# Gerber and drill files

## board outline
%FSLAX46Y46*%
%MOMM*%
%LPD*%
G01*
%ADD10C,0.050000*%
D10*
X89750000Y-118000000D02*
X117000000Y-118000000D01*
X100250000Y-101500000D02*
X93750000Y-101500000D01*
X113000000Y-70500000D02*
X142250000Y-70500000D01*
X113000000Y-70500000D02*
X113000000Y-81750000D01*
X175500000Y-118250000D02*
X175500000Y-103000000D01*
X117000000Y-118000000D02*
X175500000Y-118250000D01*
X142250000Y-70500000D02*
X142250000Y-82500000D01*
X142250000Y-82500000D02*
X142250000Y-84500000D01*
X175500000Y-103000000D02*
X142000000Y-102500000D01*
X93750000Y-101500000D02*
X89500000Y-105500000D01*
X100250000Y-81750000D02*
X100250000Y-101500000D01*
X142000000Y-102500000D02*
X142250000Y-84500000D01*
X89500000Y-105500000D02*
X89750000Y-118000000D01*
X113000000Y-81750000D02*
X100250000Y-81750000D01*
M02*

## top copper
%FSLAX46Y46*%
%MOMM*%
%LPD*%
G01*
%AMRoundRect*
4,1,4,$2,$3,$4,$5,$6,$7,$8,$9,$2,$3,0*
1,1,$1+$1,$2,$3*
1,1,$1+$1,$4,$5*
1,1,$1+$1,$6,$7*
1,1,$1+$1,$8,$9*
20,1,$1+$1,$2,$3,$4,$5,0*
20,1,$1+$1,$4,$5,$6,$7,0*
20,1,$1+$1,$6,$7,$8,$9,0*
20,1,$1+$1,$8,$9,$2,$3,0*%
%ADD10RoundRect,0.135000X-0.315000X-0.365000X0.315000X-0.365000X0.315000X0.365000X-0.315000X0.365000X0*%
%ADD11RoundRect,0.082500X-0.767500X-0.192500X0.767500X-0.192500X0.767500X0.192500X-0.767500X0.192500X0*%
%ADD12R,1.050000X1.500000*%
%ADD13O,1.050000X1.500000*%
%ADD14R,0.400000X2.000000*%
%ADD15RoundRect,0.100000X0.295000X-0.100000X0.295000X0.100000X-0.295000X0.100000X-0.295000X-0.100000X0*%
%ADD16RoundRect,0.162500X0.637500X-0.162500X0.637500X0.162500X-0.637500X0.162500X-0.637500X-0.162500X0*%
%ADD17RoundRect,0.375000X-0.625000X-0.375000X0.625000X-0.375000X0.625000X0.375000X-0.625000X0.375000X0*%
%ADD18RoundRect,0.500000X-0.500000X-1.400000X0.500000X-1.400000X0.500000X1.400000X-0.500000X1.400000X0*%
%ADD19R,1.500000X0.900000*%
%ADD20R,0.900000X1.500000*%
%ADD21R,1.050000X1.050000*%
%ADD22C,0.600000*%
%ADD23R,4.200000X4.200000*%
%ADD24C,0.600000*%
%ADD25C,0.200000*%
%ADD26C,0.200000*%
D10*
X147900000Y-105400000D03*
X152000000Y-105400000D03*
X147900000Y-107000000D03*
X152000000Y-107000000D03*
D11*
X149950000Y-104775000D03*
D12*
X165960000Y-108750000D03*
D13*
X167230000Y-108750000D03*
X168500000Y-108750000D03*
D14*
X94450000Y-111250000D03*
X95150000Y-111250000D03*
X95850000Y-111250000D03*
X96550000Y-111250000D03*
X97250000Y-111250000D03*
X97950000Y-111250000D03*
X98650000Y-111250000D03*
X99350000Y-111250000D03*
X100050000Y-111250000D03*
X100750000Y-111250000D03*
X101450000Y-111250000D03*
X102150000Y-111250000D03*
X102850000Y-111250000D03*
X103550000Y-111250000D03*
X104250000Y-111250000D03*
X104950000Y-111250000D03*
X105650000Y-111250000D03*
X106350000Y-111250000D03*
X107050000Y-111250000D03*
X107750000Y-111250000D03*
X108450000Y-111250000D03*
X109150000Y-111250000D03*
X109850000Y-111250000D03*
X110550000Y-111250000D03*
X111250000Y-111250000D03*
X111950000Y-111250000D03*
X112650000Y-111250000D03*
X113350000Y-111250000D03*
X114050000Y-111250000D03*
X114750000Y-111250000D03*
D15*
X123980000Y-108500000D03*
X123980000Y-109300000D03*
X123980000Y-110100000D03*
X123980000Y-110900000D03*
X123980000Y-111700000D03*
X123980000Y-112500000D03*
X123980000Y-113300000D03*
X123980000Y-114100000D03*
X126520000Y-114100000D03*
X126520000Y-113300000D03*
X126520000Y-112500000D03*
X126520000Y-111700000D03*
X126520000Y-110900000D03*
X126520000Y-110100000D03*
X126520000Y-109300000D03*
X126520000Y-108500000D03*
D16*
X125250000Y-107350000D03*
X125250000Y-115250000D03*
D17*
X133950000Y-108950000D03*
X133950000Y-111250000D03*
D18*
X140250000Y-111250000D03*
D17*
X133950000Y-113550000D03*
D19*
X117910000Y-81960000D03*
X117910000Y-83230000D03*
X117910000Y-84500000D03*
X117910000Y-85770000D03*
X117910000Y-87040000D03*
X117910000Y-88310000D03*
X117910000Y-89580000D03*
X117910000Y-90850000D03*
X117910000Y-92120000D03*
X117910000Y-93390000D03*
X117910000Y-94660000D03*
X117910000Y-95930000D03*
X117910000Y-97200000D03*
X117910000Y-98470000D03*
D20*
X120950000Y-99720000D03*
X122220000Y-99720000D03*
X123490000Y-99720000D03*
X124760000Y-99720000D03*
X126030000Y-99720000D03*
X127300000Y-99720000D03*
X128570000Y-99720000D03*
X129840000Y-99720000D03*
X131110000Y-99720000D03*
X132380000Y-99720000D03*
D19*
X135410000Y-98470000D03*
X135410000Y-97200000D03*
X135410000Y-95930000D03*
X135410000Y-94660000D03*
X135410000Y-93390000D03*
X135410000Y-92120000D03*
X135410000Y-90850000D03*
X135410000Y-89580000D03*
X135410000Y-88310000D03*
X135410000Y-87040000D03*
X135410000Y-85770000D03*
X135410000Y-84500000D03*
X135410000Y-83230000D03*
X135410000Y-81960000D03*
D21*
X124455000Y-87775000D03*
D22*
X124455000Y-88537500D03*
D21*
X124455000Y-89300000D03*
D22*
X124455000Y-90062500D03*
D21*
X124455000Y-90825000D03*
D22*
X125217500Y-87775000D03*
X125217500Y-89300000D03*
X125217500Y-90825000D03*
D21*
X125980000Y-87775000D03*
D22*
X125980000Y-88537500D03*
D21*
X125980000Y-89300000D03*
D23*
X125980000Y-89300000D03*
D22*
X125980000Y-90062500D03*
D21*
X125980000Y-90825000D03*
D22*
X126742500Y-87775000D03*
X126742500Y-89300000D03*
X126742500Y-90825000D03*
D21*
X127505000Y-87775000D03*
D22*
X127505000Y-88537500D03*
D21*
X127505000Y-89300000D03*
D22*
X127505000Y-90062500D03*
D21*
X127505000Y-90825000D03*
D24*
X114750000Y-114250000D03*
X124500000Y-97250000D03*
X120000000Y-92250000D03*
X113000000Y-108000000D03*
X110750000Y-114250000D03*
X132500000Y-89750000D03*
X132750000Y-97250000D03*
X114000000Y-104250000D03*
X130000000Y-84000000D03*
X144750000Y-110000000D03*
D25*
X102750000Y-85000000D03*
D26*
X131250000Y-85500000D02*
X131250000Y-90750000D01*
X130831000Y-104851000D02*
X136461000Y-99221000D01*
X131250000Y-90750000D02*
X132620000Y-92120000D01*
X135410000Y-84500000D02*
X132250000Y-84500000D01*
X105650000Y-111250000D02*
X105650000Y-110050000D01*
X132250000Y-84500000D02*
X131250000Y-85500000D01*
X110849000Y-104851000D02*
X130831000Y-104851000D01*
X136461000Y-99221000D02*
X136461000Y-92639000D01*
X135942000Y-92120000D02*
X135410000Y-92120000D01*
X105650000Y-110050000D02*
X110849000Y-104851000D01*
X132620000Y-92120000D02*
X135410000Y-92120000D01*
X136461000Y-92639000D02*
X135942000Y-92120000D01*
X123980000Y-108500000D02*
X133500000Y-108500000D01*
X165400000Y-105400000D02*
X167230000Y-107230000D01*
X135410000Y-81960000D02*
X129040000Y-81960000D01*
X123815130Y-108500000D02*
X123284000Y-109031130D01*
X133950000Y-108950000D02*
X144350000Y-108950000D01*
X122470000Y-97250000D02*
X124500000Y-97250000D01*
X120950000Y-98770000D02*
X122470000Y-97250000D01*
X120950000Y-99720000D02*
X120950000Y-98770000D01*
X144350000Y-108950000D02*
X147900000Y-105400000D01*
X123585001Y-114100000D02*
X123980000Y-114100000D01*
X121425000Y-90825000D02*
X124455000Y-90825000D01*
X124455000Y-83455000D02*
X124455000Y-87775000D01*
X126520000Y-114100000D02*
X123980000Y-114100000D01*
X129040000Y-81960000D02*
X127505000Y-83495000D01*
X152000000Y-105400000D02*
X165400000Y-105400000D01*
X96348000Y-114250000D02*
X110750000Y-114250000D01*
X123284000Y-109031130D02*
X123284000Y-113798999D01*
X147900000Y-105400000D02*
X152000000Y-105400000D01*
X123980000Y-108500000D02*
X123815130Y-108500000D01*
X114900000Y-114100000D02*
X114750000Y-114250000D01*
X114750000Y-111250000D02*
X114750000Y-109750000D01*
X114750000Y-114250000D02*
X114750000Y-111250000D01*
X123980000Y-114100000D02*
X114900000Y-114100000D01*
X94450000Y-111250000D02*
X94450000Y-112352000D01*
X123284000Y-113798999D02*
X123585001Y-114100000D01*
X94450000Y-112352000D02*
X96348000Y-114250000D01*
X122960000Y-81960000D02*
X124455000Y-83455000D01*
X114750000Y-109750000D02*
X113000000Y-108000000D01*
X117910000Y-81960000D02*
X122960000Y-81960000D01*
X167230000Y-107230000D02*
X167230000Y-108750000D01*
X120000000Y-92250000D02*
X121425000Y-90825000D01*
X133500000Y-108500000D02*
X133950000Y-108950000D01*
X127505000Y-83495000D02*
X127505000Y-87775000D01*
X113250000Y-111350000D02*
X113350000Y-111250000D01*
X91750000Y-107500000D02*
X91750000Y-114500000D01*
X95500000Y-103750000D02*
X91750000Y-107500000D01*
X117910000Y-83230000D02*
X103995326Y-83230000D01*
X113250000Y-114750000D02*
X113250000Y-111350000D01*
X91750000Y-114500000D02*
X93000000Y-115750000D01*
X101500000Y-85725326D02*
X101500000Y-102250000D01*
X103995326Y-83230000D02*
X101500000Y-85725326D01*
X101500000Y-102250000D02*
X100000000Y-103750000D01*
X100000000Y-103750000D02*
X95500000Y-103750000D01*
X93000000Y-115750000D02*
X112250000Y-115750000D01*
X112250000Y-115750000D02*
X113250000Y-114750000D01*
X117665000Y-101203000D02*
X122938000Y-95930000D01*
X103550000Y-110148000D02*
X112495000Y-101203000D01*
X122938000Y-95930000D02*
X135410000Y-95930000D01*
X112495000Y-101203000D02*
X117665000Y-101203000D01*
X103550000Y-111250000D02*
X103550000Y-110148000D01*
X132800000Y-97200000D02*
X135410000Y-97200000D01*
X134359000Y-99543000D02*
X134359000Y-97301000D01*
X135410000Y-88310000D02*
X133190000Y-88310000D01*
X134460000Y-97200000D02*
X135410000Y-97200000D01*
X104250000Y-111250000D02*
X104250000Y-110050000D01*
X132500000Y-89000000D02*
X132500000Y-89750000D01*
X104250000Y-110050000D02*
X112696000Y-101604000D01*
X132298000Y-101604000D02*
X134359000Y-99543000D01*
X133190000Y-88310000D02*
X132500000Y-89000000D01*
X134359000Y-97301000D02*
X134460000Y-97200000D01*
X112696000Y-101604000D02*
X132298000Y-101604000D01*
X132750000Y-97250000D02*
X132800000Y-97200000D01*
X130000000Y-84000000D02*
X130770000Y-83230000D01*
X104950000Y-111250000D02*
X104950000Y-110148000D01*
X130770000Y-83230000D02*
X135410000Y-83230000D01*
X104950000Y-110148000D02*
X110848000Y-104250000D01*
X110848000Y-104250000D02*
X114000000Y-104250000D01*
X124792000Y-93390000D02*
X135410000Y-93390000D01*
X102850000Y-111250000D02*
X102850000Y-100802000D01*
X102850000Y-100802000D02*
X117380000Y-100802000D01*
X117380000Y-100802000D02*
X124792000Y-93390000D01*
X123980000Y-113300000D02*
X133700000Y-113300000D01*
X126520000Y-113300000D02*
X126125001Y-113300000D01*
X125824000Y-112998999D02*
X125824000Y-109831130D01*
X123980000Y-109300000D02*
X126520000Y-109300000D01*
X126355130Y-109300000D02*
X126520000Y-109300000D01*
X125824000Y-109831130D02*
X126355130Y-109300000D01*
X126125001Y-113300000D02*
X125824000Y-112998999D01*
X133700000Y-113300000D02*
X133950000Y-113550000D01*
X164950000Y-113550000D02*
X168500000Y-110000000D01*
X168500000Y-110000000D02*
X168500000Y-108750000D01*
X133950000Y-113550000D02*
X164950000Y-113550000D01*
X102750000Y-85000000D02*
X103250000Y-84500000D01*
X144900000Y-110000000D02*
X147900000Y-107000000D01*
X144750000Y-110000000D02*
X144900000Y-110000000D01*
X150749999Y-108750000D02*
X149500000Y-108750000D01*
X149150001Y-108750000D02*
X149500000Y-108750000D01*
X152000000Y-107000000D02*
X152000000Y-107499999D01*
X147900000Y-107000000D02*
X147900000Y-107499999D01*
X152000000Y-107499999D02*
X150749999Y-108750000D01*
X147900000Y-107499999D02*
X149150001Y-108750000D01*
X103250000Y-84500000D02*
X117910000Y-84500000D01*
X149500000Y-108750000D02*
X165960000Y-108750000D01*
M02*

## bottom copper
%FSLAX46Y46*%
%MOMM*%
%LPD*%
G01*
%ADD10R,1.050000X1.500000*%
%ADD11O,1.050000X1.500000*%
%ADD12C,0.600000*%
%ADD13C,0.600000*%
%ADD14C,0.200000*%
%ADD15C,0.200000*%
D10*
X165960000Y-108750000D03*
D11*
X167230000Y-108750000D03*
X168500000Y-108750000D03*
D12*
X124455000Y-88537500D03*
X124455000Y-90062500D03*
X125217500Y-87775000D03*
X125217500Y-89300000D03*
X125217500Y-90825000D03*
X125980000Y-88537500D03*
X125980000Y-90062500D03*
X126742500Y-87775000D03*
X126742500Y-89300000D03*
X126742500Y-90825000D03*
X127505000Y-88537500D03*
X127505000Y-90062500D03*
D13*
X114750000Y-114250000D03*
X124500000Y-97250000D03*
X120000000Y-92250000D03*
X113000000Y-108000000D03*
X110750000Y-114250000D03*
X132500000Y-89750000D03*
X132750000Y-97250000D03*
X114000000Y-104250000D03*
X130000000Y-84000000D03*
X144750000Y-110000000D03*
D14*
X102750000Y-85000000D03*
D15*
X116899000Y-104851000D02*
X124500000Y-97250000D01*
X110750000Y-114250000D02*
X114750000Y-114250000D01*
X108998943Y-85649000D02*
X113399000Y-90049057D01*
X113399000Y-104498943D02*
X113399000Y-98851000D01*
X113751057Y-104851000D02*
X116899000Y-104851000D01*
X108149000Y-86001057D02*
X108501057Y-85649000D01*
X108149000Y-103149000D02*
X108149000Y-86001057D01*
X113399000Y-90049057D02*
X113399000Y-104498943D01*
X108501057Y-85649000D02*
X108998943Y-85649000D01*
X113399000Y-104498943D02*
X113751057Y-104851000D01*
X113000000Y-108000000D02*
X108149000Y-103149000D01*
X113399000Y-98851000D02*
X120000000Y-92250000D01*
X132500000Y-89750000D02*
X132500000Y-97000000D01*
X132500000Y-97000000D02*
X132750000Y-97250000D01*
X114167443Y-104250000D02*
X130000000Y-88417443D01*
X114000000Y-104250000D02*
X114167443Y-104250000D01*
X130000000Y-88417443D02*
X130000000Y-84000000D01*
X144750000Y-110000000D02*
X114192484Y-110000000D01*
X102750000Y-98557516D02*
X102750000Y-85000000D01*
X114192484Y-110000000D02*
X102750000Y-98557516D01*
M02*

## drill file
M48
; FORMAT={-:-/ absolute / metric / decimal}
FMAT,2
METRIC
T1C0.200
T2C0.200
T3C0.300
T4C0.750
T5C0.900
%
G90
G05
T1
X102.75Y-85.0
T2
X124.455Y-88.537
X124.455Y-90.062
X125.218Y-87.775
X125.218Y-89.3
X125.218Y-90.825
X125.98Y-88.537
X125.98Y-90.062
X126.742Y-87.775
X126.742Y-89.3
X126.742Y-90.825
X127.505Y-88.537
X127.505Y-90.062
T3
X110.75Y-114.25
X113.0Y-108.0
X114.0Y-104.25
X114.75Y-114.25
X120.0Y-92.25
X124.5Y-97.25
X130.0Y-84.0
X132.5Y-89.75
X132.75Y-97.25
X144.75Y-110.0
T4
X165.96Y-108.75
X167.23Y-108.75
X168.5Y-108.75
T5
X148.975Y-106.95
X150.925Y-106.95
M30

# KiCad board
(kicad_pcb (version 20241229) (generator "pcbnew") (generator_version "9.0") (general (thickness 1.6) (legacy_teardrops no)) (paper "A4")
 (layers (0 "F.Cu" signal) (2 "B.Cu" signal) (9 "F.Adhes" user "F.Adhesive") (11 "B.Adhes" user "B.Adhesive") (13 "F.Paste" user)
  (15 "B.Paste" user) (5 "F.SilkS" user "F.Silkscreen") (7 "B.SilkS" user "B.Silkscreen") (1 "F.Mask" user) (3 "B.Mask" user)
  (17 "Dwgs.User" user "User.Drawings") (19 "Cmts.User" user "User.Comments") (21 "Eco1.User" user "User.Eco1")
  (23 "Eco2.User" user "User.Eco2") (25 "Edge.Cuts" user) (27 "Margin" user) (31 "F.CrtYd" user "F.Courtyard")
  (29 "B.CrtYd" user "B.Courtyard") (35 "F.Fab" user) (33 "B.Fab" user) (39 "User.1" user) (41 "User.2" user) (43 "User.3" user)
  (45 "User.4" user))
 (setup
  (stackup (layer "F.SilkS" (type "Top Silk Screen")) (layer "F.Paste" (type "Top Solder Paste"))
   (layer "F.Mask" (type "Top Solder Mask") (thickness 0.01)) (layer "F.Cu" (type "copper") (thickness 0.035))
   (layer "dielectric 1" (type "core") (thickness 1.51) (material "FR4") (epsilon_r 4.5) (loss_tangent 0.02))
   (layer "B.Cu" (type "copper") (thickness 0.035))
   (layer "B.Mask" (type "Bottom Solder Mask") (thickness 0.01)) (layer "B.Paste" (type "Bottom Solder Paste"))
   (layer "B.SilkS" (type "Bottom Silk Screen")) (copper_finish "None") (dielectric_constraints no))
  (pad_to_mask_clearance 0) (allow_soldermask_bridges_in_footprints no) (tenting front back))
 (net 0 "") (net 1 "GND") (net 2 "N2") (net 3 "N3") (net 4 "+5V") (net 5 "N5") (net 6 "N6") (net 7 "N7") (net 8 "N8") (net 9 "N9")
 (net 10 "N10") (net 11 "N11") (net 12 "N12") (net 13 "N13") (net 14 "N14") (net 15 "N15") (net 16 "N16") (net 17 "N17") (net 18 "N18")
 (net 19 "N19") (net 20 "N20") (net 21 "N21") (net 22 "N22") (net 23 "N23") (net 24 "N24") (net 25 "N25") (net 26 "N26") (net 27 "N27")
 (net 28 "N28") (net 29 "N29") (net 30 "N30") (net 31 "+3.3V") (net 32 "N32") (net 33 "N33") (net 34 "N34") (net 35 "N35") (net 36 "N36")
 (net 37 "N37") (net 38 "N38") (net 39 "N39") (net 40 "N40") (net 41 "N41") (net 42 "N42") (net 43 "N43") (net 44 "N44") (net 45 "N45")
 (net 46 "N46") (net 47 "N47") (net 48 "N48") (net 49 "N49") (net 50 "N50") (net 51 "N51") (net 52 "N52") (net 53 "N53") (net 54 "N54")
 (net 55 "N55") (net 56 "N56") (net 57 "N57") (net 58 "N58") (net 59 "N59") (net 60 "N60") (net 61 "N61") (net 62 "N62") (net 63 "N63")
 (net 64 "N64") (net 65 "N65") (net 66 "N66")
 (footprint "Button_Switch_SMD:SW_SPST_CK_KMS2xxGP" (layer "F.Cu") (at 149.95 106.2)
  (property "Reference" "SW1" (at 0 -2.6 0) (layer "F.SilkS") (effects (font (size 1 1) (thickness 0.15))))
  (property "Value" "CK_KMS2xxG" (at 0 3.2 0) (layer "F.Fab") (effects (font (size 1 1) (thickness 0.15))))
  (pad "" np_thru_hole circle (at -0.975 0.75) (size 0.9 0.9) (drill 0.9) (layers "*.Cu" "*.Mask"))
  (pad "" np_thru_hole circle (at 0.975 0.75) (size 0.9 0.9) (drill 0.9) (layers "*.Cu" "*.Mask"))
  (pad "1" smd roundrect (at -2.05 -0.8) (size 0.9 1) (layers "F.Cu" "F.Mask" "F.Paste") (roundrect_rratio 0.15) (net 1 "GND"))
  (pad "1" smd roundrect (at 2.05 -0.8) (size 0.9 1) (layers "F.Cu" "F.Mask" "F.Paste") (roundrect_rratio 0.15) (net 1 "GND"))
  (pad "2" smd roundrect (at -2.05 0.8) (size 0.9 1) (layers "F.Cu" "F.Mask" "F.Paste") (roundrect_rratio 0.15) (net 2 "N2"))
  (pad "2" smd roundrect (at 2.05 0.8) (size 0.9 1) (layers "F.Cu" "F.Mask" "F.Paste") (roundrect_rratio 0.15) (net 2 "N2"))
  (pad "SH" smd roundrect (at 0 -1.425) (size 1.7 0.55) (layers "F.Cu" "F.Mask" "F.Paste") (roundrect_rratio 0.15) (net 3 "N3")))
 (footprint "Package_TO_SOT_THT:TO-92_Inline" (layer "F.Cu") (at 165.96 108.75)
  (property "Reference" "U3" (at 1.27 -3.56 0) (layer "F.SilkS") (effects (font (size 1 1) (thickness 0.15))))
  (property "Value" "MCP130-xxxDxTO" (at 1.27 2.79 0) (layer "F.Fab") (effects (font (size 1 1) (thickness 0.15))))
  (pad "1" thru_hole rect (at 0 0) (size 1.05 1.5) (drill 0.75) (layers "*.Cu" "*.Mask") (remove_unused_layers no) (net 2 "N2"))
  (pad "2" thru_hole oval (at 1.27 0) (size 1.05 1.5) (drill 0.75) (layers "*.Cu" "*.Mask") (remove_unused_layers no) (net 1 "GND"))
  (pad "3" thru_hole oval (at 2.54 0) (size 1.05 1.5) (drill 0.75) (layers "*.Cu" "*.Mask") (remove_unused_layers no) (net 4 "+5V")))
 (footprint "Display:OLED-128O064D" (layer "F.Cu") (at 104.6 111.25)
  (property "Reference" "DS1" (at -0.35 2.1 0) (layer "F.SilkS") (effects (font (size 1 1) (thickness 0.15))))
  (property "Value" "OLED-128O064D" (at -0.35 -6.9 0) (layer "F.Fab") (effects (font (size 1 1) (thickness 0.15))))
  (pad "1" smd rect (at -10.15 0) (size 0.4 2) (layers "F.Cu" "F.Mask" "F.Paste") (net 1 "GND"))
  (pad "2" smd rect (at -9.45 0) (size 0.4 2) (layers "F.Cu" "F.Mask" "F.Paste") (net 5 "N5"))
  (pad "3" smd rect (at -8.75 0) (size 0.4 2) (layers "F.Cu" "F.Mask" "F.Paste") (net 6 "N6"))
  (pad "4" smd rect (at -8.05 0) (size 0.4 2) (layers "F.Cu" "F.Mask" "F.Paste") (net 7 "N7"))
  (pad "5" smd rect (at -7.35 0) (size 0.4 2) (layers "F.Cu" "F.Mask" "F.Paste") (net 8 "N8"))
  (pad "6" smd rect (at -6.65 0) (size 0.4 2) (layers "F.Cu" "F.Mask" "F.Paste") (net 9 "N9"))
  (pad "7" smd rect (at -5.95 0) (size 0.4 2) (layers "F.Cu" "F.Mask" "F.Paste") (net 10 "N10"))
  (pad "8" smd rect (at -5.25 0) (size 0.4 2) (layers "F.Cu" "F.Mask" "F.Paste") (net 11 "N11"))
  (pad "9" smd rect (at -4.55 0) (size 0.4 2) (layers "F.Cu" "F.Mask" "F.Paste") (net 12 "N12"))
  (pad "10" smd rect (at -3.85 0) (size 0.4 2) (layers "F.Cu" "F.Mask" "F.Paste") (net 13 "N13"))
  (pad "11" smd rect (at -3.15 0) (size 0.4 2) (layers "F.Cu" "F.Mask" "F.Paste") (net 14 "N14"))
  (pad "12" smd rect (at -2.45 0) (size 0.4 2) (layers "F.Cu" "F.Mask" "F.Paste") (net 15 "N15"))
  (pad "13" smd rect (at -1.75 0) (size 0.4 2) (layers "F.Cu" "F.Mask" "F.Paste") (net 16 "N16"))
  (pad "14" smd rect (at -1.05 0) (size 0.4 2) (layers "F.Cu" "F.Mask" "F.Paste") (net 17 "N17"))
  (pad "15" smd rect (at -0.35 0) (size 0.4 2) (layers "F.Cu" "F.Mask" "F.Paste") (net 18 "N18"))
  (pad "16" smd rect (at 0.35 0) (size 0.4 2) (layers "F.Cu" "F.Mask" "F.Paste") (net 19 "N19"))
  (pad "17" smd rect (at 1.05 0) (size 0.4 2) (layers "F.Cu" "F.Mask" "F.Paste") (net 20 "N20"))
  (pad "18" smd rect (at 1.75 0) (size 0.4 2) (layers "F.Cu" "F.Mask" "F.Paste") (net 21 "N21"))
  (pad "19" smd rect (at 2.45 0) (size 0.4 2) (layers "F.Cu" "F.Mask" "F.Paste") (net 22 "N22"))
  (pad "20" smd rect (at 3.15 0) (size 0.4 2) (layers "F.Cu" "F.Mask" "F.Paste") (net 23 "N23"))
  (pad "21" smd rect (at 3.85 0) (size 0.4 2) (layers "F.Cu" "F.Mask" "F.Paste") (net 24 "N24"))
  (pad "22" smd rect (at 4.55 0) (size 0.4 2) (layers "F.Cu" "F.Mask" "F.Paste") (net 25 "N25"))
  (pad "23" smd rect (at 5.25 0) (size 0.4 2) (layers "F.Cu" "F.Mask" "F.Paste") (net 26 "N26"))
  (pad "24" smd rect (at 5.95 0) (size 0.4 2) (layers "F.Cu" "F.Mask" "F.Paste") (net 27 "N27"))
  (pad "25" smd rect (at 6.65 0) (size 0.4 2) (layers "F.Cu" "F.Mask" "F.Paste") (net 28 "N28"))
  (pad "26" smd rect (at 7.35 0) (size 0.4 2) (layers "F.Cu" "F.Mask" "F.Paste") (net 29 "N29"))
  (pad "27" smd rect (at 8.05 0) (size 0.4 2) (layers "F.Cu" "F.Mask" "F.Paste") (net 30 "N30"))
  (pad "28" smd rect (at 8.75 0) (size 0.4 2) (layers "F.Cu" "F.Mask" "F.Paste") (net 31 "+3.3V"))
  (pad "29" smd rect (at 9.45 0) (size 0.4 2) (layers "F.Cu" "F.Mask" "F.Paste") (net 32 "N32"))
  (pad "30" smd rect (at 10.15 0) (size 0.4 2) (layers "F.Cu" "F.Mask" "F.Paste") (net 1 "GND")))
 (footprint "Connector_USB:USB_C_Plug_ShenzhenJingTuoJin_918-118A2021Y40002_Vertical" (layer "F.Cu") (at 125.25 111.3)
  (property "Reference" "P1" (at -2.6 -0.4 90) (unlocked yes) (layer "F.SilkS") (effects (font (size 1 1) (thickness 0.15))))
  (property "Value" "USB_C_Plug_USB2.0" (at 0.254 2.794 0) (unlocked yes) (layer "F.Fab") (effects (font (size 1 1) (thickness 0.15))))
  (pad "A1" smd roundrect (at -1.27 -2.8 90) (size 0.4 0.79) (layers "F.Cu" "F.Mask" "F.Paste") (roundrect_rratio 0.25) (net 1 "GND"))
  (pad "A4" smd roundrect (at -1.27 -2 90) (size 0.4 0.79) (layers "F.Cu" "F.Mask" "F.Paste") (roundrect_rratio 0.25) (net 4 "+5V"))
  (pad "A5" smd roundrect (at -1.27 -1.2 90) (size 0.4 0.79) (layers "F.Cu" "F.Mask" "F.Paste") (roundrect_rratio 0.25) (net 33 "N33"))
  (pad "A6" smd roundrect (at -1.27 -0.4 90) (size 0.4 0.79) (layers "F.Cu" "F.Mask" "F.Paste") (roundrect_rratio 0.25) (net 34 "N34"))
  (pad "A7" smd roundrect (at -1.27 0.4 90) (size 0.4 0.79) (layers "F.Cu" "F.Mask" "F.Paste") (roundrect_rratio 0.25) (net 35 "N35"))
  (pad "A8" smd roundrect (at -1.27 1.2 90) (size 0.4 0.79) (layers "F.Cu" "F.Mask" "F.Paste") (roundrect_rratio 0.25))
  (pad "A9" smd roundrect (at -1.27 2 90) (size 0.4 0.79) (layers "F.Cu" "F.Mask" "F.Paste") (roundrect_rratio 0.25) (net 4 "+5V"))
  (pad "A12" smd roundrect (at -1.27 2.8 90) (size 0.4 0.79) (layers "F.Cu" "F.Mask" "F.Paste") (roundrect_rratio 0.25) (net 1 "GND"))
  (pad "B1" smd roundrect (at 1.27 2.8 90) (size 0.4 0.79) (layers "F.Cu" "F.Mask" "F.Paste") (roundrect_rratio 0.25) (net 1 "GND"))
  (pad "B4" smd roundrect (at 1.27 2 90) (size 0.4 0.79) (layers "F.Cu" "F.Mask" "F.Paste") (roundrect_rratio 0.25) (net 4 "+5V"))
  (pad "B5" smd roundrect (at 1.27 1.2 90) (size 0.4 0.79) (layers "F.Cu" "F.Mask" "F.Paste") (roundrect_rratio 0.25) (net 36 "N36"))
  (pad "B6" smd roundrect (at 1.27 0.4 90) (size 0.4 0.79) (layers "F.Cu" "F.Mask" "F.Paste") (roundrect_rratio 0.25))
  (pad "B7" smd roundrect (at 1.27 -0.4 90) (size 0.4 0.79) (layers "F.Cu" "F.Mask" "F.Paste") (roundrect_rratio 0.25))
  (pad "B8" smd roundrect (at 1.27 -1.2 90) (size 0.4 0.79) (layers "F.Cu" "F.Mask" "F.Paste") (roundrect_rratio 0.25))
  (pad "B9" smd roundrect (at 1.27 -2 90) (size 0.4 0.79) (layers "F.Cu" "F.Mask" "F.Paste") (roundrect_rratio 0.25) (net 4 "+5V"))
  (pad "B12" smd roundrect (at 1.27 -2.8 90) (size 0.4 0.79) (layers "F.Cu" "F.Mask" "F.Paste") (roundrect_rratio 0.25) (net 1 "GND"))
  (pad "S1" smd roundrect (at 0 -3.95 90) (size 0.65 1.6) (layers "F.Cu" "F.Mask" "F.Paste") (roundrect_rratio 0.25) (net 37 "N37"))
  (pad "S1" smd roundrect (at 0 3.95 90) (size 0.65 1.6) (layers "F.Cu" "F.Mask" "F.Paste") (roundrect_rratio 0.25) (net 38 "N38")))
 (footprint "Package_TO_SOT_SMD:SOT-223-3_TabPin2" (layer "F.Cu") (at 137.1 111.25)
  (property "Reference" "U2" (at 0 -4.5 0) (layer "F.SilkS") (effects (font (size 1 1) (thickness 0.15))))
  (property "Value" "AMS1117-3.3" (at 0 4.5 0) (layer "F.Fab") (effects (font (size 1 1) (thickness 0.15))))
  (pad "1" smd roundrect (at -3.15 -2.3) (size 2 1.5) (layers "F.Cu" "F.Mask" "F.Paste") (roundrect_rratio 0.25) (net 1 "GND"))
  (pad "2" smd roundrect (at -3.15 0) (size 2 1.5) (layers "F.Cu" "F.Mask" "F.Paste") (roundrect_rratio 0.25) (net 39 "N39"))
  (pad "2" smd roundrect (at 3.15 0) (size 2 3.8) (layers "F.Cu" "F.Mask" "F.Paste") (roundrect_rratio 0.25) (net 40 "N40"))
  (pad "3" smd roundrect (at -3.15 2.3) (size 2 1.5) (layers "F.Cu" "F.Mask" "F.Paste") (roundrect_rratio 0.25) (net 4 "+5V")))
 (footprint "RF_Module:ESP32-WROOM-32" (layer "F.Cu") (at 126.66 90.21)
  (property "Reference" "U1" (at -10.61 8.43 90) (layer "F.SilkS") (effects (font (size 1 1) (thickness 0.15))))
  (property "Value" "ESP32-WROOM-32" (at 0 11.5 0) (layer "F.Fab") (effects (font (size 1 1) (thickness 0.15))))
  (pad "1" smd rect (at -8.75 -8.25) (size 1.5 0.9) (layers "F.Cu" "F.Mask" "F.Paste") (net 1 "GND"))
  (pad "2" smd rect (at -8.75 -6.98) (size 1.5 0.9) (layers "F.Cu" "F.Mask" "F.Paste") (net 31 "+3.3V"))
  (pad "3" smd rect (at -8.75 -5.71) (size 1.5 0.9) (layers "F.Cu" "F.Mask" "F.Paste") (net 2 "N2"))
  (pad "4" smd rect (at -8.75 -4.44) (size 1.5 0.9) (layers "F.Cu" "F.Mask" "F.Paste") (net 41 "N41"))
  (pad "5" smd rect (at -8.75 -3.17) (size 1.5 0.9) (layers "F.Cu" "F.Mask" "F.Paste") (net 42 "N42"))
  (pad "6" smd rect (at -8.75 -1.9) (size 1.5 0.9) (layers "F.Cu" "F.Mask" "F.Paste") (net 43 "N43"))
  (pad "7" smd rect (at -8.75 -0.63) (size 1.5 0.9) (layers "F.Cu" "F.Mask" "F.Paste") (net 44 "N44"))
  (pad "8" smd rect (at -8.75 0.64) (size 1.5 0.9) (layers "F.Cu" "F.Mask" "F.Paste") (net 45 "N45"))
  (pad "9" smd rect (at -8.75 1.91) (size 1.5 0.9) (layers "F.Cu" "F.Mask" "F.Paste") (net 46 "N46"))
  (pad "10" smd rect (at -8.75 3.18) (size 1.5 0.9) (layers "F.Cu" "F.Mask" "F.Paste") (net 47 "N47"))
  (pad "11" smd rect (at -8.75 4.45) (size 1.5 0.9) (layers "F.Cu" "F.Mask" "F.Paste") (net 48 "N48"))
  (pad "12" smd rect (at -8.75 5.72) (size 1.5 0.9) (layers "F.Cu" "F.Mask" "F.Paste") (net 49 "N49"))
  (pad "13" smd rect (at -8.75 6.99) (size 1.5 0.9) (layers "F.Cu" "F.Mask" "F.Paste") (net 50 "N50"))
  (pad "14" smd rect (at -8.75 8.26) (size 1.5 0.9) (layers "F.Cu" "F.Mask" "F.Paste") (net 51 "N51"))
  (pad "15" smd rect (at -5.71 9.51 90) (size 1.5 0.9) (layers "F.Cu" "F.Mask" "F.Paste") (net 1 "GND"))
  (pad "16" smd rect (at -4.44 9.51 90) (size 1.5 0.9) (layers "F.Cu" "F.Mask" "F.Paste") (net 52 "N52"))
  (pad "17" smd rect (at -3.17 9.51 90) (size 1.5 0.9) (layers "F.Cu" "F.Mask" "F.Paste") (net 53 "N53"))
  (pad "18" smd rect (at -1.9 9.51 90) (size 1.5 0.9) (layers "F.Cu" "F.Mask" "F.Paste") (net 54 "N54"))
  (pad "19" smd rect (at -0.63 9.51 90) (size 1.5 0.9) (layers "F.Cu" "F.Mask" "F.Paste") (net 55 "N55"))
  (pad "20" smd rect (at 0.64 9.51 90) (size 1.5 0.9) (layers "F.Cu" "F.Mask" "F.Paste") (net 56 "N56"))
  (pad "21" smd rect (at 1.91 9.51 90) (size 1.5 0.9) (layers "F.Cu" "F.Mask" "F.Paste") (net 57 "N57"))
  (pad "22" smd rect (at 3.18 9.51 90) (size 1.5 0.9) (layers "F.Cu" "F.Mask" "F.Paste") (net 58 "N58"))
  (pad "23" smd rect (at 4.45 9.51 90) (size 1.5 0.9) (layers "F.Cu" "F.Mask" "F.Paste") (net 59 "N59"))
  (pad "24" smd rect (at 5.72 9.51 90) (size 1.5 0.9) (layers "F.Cu" "F.Mask" "F.Paste") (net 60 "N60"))
  (pad "25" smd rect (at 8.75 8.26) (size 1.5 0.9) (layers "F.Cu" "F.Mask" "F.Paste") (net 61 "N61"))
  (pad "26" smd rect (at 8.75 6.99) (size 1.5 0.9) (layers "F.Cu" "F.Mask" "F.Paste") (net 18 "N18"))
  (pad "27" smd rect (at 8.75 5.72) (size 1.5 0.9) (layers "F.Cu" "F.Mask" "F.Paste") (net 17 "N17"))
  (pad "28" smd rect (at 8.75 4.45) (size 1.5 0.9) (layers "F.Cu" "F.Mask" "F.Paste") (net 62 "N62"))
  (pad "29" smd rect (at 8.75 3.18) (size 1.5 0.9) (layers "F.Cu" "F.Mask" "F.Paste") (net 16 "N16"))
  (pad "30" smd rect (at 8.75 1.91) (size 1.5 0.9) (layers "F.Cu" "F.Mask" "F.Paste") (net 20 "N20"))
  (pad "31" smd rect (at 8.75 0.64) (size 1.5 0.9) (layers "F.Cu" "F.Mask" "F.Paste") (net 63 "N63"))
  (pad "32" smd rect (at 8.75 -0.63) (size 1.5 0.9) (layers "F.Cu" "F.Mask" "F.Paste") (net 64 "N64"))
  (pad "33" smd rect (at 8.75 -1.9) (size 1.5 0.9) (layers "F.Cu" "F.Mask" "F.Paste") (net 18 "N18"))
  (pad "34" smd rect (at 8.75 -3.17) (size 1.5 0.9) (layers "F.Cu" "F.Mask" "F.Paste") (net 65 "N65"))
  (pad "35" smd rect (at 8.75 -4.44) (size 1.5 0.9) (layers "F.Cu" "F.Mask" "F.Paste") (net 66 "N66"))
  (pad "36" smd rect (at 8.75 -5.71) (size 1.5 0.9) (layers "F.Cu" "F.Mask" "F.Paste") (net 20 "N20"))
  (pad "37" smd rect (at 8.75 -6.98) (size 1.5 0.9) (layers "F.Cu" "F.Mask" "F.Paste") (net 19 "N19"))
  (pad "38" smd rect (at 8.75 -8.25) (size 1.5 0.9) (layers "F.Cu" "F.Mask" "F.Paste") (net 1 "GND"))
  (pad "39" smd rect (at -2.205 -2.435) (size 1.05 1.05) (layers "F.Cu" "F.Paste") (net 1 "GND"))
  (pad "39" thru_hole circle (at -2.205 -1.6725) (size 0.6 0.6) (drill 0.2) (layers "*.Cu" "F.Mask") (remove_unused_layers no) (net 1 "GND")
   (zone_connect 2))
  (pad "39" smd rect (at -2.205 -0.91) (size 1.05 1.05) (layers "F.Cu" "F.Paste") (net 1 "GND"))
  (pad "39" thru_hole circle (at -2.205 -0.1475) (size 0.6 0.6) (drill 0.2) (layers "*.Cu" "F.Mask") (remove_unused_layers no) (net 1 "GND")
   (zone_connect 2))
  (pad "39" smd rect (at -2.205 0.615) (size 1.05 1.05) (layers "F.Cu" "F.Paste") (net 1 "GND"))
  (pad "39" thru_hole circle (at -1.4425 -2.435) (size 0.6 0.6) (drill 0.2) (layers "*.Cu" "F.Mask") (remove_unused_layers no) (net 1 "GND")
   (zone_connect 2))
  (pad "39" thru_hole circle (at -1.4425 -0.91) (size 0.6 0.6) (drill 0.2) (layers "*.Cu" "F.Mask") (remove_unused_layers no) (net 1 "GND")
   (zone_connect 2))
  (pad "39" thru_hole circle (at -1.4425 0.615) (size 0.6 0.6) (drill 0.2) (layers "*.Cu" "F.Mask") (remove_unused_layers no) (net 1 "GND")
   (zone_connect 2))
  (pad "39" smd rect (at -0.68 -2.435) (size 1.05 1.05) (layers "F.Cu" "F.Paste") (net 1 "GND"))
  (pad "39" thru_hole circle (at -0.68 -1.6725) (size 0.6 0.6) (drill 0.2) (layers "*.Cu" "F.Mask") (remove_unused_layers no) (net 1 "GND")
   (zone_connect 2))
  (pad "39" smd rect (at -0.68 -0.91) (size 1.05 1.05) (layers "F.Cu" "F.Paste") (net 1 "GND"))
  (pad "39" smd rect (at -0.68 -0.91) (size 4.2 4.2) (layers "F.Cu" "F.Mask") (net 1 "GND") (zone_connect 2))
  (pad "39" thru_hole circle (at -0.68 -0.1475) (size 0.6 0.6) (drill 0.2) (layers "*.Cu" "F.Mask") (remove_unused_layers no) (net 1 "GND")
   (zone_connect 2))
  (pad "39" smd rect (at -0.68 0.615) (size 1.05 1.05) (layers "F.Cu" "F.Paste") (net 1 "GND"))
  (pad "39" thru_hole circle (at 0.0825 -2.435) (size 0.6 0.6) (drill 0.2) (layers "*.Cu" "F.Mask") (remove_unused_layers no) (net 1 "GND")
   (zone_connect 2))
  (pad "39" thru_hole circle (at 0.0825 -0.91) (size 0.6 0.6) (drill 0.2) (layers "*.Cu" "F.Mask") (remove_unused_layers no) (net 1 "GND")
   (zone_connect 2))
  (pad "39" thru_hole circle (at 0.0825 0.615) (size 0.6 0.6) (drill 0.2) (layers "*.Cu" "F.Mask") (remove_unused_layers no) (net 1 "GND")
   (zone_connect 2))
  (pad "39" smd rect (at 0.845 -2.435) (size 1.05 1.05) (layers "F.Cu" "F.Paste") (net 1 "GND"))
  (pad "39" thru_hole circle (at 0.845 -1.6725) (size 0.6 0.6) (drill 0.2) (layers "*.Cu" "F.Mask") (remove_unused_layers no) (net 1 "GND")
   (zone_connect 2))
  (pad "39" smd rect (at 0.845 -0.91) (size 1.05 1.05) (layers "F.Cu" "F.Paste") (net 1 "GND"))
  (pad "39" thru_hole circle (at 0.845 -0.1475) (size 0.6 0.6) (drill 0.2) (layers "*.Cu" "F.Mask") (remove_unused_layers no) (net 1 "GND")
   (zone_connect 2))
  (pad "39" smd rect (at 0.845 0.615) (size 1.05 1.05) (layers "F.Cu" "F.Paste") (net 1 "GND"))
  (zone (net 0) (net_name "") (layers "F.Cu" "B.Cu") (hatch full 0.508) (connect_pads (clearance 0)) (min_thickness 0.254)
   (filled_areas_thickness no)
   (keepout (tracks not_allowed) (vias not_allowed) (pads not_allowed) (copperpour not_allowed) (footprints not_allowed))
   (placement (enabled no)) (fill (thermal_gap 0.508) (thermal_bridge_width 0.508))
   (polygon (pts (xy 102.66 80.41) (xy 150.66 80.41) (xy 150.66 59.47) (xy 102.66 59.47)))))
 (gr_line (start 89.75 118) (end 117 118) (stroke (width 0.05) (type default)) (layer "Edge.Cuts"))
 (gr_line (start 100.25 101.5) (end 93.75 101.5) (stroke (width 0.05) (type default)) (layer "Edge.Cuts"))
 (gr_line (start 113 70.5) (end 142.25 70.5) (stroke (width 0.05) (type default)) (layer "Edge.Cuts"))
 (gr_line (start 113 70.5) (end 113 81.75) (stroke (width 0.05) (type default)) (layer "Edge.Cuts"))
 (gr_line (start 175.5 118.25) (end 175.5 103) (stroke (width 0.05) (type default)) (layer "Edge.Cuts"))
 (gr_line (start 117 118) (end 175.5 118.25) (stroke (width 0.05) (type default)) (layer "Edge.Cuts"))
 (gr_line (start 142.25 70.5) (end 142.25 82.5) (stroke (width 0.05) (type default)) (layer "Edge.Cuts"))
 (gr_line (start 142.25 82.5) (end 142.25 84.5) (stroke (width 0.05) (type default)) (layer "Edge.Cuts"))
 (gr_line (start 175.5 103) (end 142 102.5) (stroke (width 0.05) (type default)) (layer "Edge.Cuts"))
 (gr_line (start 93.75 101.5) (end 89.5 105.5) (stroke (width 0.05) (type default)) (layer "Edge.Cuts"))
 (gr_line (start 100.25 81.75) (end 100.25 101.5) (stroke (width 0.05) (type default)) (layer "Edge.Cuts"))
 (gr_line (start 142 102.5) (end 142.25 84.5) (stroke (width 0.05) (type default)) (layer "Edge.Cuts"))
 (gr_line (start 89.5 105.5) (end 89.75 118) (stroke (width 0.05) (type default)) (layer "Edge.Cuts"))
 (gr_line (start 113 81.75) (end 100.25 81.75) (stroke (width 0.05) (type default)) (layer "Edge.Cuts"))
 (segment (start 131.25 85.5) (end 131.25 90.75) (width 0.2) (layer "F.Cu") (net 20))
 (segment (start 130.831 104.851) (end 136.461 99.221) (width 0.2) (layer "F.Cu") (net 20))
 (segment (start 131.25 90.75) (end 132.62 92.12) (width 0.2) (layer "F.Cu") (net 20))
 (segment (start 135.41 84.5) (end 132.25 84.5) (width 0.2) (layer "F.Cu") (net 20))
 (segment (start 105.65 111.25) (end 105.65 110.05) (width 0.2) (layer "F.Cu") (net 20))
 (segment (start 132.25 84.5) (end 131.25 85.5) (width 0.2) (layer "F.Cu") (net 20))
 (segment (start 110.849 104.851) (end 130.831 104.851) (width 0.2) (layer "F.Cu") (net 20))
 (segment (start 136.461 99.221) (end 136.461 92.639) (width 0.2) (layer "F.Cu") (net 20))
 (segment (start 135.942 92.12) (end 135.41 92.12) (width 0.2) (layer "F.Cu") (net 20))
 (segment (start 105.65 110.05) (end 110.849 104.851) (width 0.2) (layer "F.Cu") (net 20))
 (segment (start 132.62 92.12) (end 135.41 92.12) (width 0.2) (layer "F.Cu") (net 20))
 (segment (start 136.461 92.639) (end 135.942 92.12) (width 0.2) (layer "F.Cu") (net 20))
 (segment (start 123.98 108.5) (end 133.5 108.5) (width 0.2) (layer "F.Cu") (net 1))
 (segment (start 165.4 105.4) (end 167.23 107.23) (width 0.2) (layer "F.Cu") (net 1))
 (segment (start 135.41 81.96) (end 129.04 81.96) (width 0.2) (layer "F.Cu") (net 1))
 (segment (start 123.81513 108.5) (end 123.284 109.03113) (width 0.2) (layer "F.Cu") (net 1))
 (segment (start 133.95 108.95) (end 144.35 108.95) (width 0.2) (layer "F.Cu") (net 1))
 (segment (start 122.47 97.25) (end 124.5 97.25) (width 0.2) (layer "F.Cu") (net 1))
 (segment (start 120.95 98.77) (end 122.47 97.25) (width 0.2) (layer "F.Cu") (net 1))
 (segment (start 120.95 99.72) (end 120.95 98.77) (width 0.2) (layer "F.Cu") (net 1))
 (segment (start 144.35 108.95) (end 147.9 105.4) (width 0.2) (layer "F.Cu") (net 1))
 (segment (start 123.585001 114.1) (end 123.98 114.1) (width 0.2) (layer "F.Cu") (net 1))
 (segment (start 121.425 90.825) (end 124.455 90.825) (width 0.2) (layer "F.Cu") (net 1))
 (segment (start 124.455 83.455) (end 124.455 87.775) (width 0.2) (layer "F.Cu") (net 1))
 (segment (start 126.52 114.1) (end 123.98 114.1) (width 0.2) (layer "F.Cu") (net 1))
 (segment (start 129.04 81.96) (end 127.505 83.495) (width 0.2) (layer "F.Cu") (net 1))
 (segment (start 152 105.4) (end 165.4 105.4) (width 0.2) (layer "F.Cu") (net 1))
 (segment (start 96.348 114.25) (end 110.75 114.25) (width 0.2) (layer "F.Cu") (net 1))
 (segment (start 123.284 109.03113) (end 123.284 113.798999) (width 0.2) (layer "F.Cu") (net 1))
 (segment (start 147.9 105.4) (end 152 105.4) (width 0.2) (layer "F.Cu") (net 1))
 (segment (start 123.98 108.5) (end 123.81513 108.5) (width 0.2) (layer "F.Cu") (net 1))
 (segment (start 114.9 114.1) (end 114.75 114.25) (width 0.2) (layer "F.Cu") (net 1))
 (segment (start 114.75 111.25) (end 114.75 109.75) (width 0.2) (layer "F.Cu") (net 1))
 (segment (start 114.75 114.25) (end 114.75 111.25) (width 0.2) (layer "F.Cu") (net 1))
 (segment (start 123.98 114.1) (end 114.9 114.1) (width 0.2) (layer "F.Cu") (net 1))
 (segment (start 94.45 111.25) (end 94.45 112.352) (width 0.2) (layer "F.Cu") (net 1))
 (segment (start 123.284 113.798999) (end 123.585001 114.1) (width 0.2) (layer "F.Cu") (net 1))
 (segment (start 94.45 112.352) (end 96.348 114.25) (width 0.2) (layer "F.Cu") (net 1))
 (segment (start 122.96 81.96) (end 124.455 83.455) (width 0.2) (layer "F.Cu") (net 1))
 (segment (start 114.75 109.75) (end 113 108) (width 0.2) (layer "F.Cu") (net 1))
 (segment (start 117.91 81.96) (end 122.96 81.96) (width 0.2) (layer "F.Cu") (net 1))
 (segment (start 167.23 107.23) (end 167.23 108.75) (width 0.2) (layer "F.Cu") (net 1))
 (segment (start 120 92.25) (end 121.425 90.825) (width 0.2) (layer "F.Cu") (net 1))
 (segment (start 133.5 108.5) (end 133.95 108.95) (width 0.2) (layer "F.Cu") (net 1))
 (segment (start 127.505 83.495) (end 127.505 87.775) (width 0.2) (layer "F.Cu") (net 1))
 (via (at 114.75 114.25) (size 0.6) (drill 0.3) (layers "F.Cu" "B.Cu") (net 1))
 (via (at 124.5 97.25) (size 0.6) (drill 0.3) (layers "F.Cu" "B.Cu") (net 1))
 (via (at 120 92.25) (size 0.6) (drill 0.3) (layers "F.Cu" "B.Cu") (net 1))
 (via (at 113 108) (size 0.6) (drill 0.3) (layers "F.Cu" "B.Cu") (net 1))
 (via (at 110.75 114.25) (size 0.6) (drill 0.3) (layers "F.Cu" "B.Cu") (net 1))
 (segment (start 116.899 104.851) (end 124.5 97.25) (width 0.2) (layer "B.Cu") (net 1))
 (segment (start 110.75 114.25) (end 114.75 114.25) (width 0.2) (layer "B.Cu") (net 1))
 (segment (start 108.998943 85.649) (end 113.399 90.049057) (width 0.2) (layer "B.Cu") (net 1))
 (segment (start 113.399 104.498943) (end 113.399 98.851) (width 0.2) (layer "B.Cu") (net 1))
 (segment (start 113.751057 104.851) (end 116.899 104.851) (width 0.2) (layer "B.Cu") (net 1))
 (segment (start 108.149 86.001057) (end 108.501057 85.649) (width 0.2) (layer "B.Cu") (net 1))
 (segment (start 108.149 103.149) (end 108.149 86.001057) (width 0.2) (layer "B.Cu") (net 1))
 (segment (start 113.399 90.049057) (end 113.399 104.498943) (width 0.2) (layer "B.Cu") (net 1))
 (segment (start 108.501057 85.649) (end 108.998943 85.649) (width 0.2) (layer "B.Cu") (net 1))
 (segment (start 113.399 104.498943) (end 113.751057 104.851) (width 0.2) (layer "B.Cu") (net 1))
 (segment (start 113 108) (end 108.149 103.149) (width 0.2) (layer "B.Cu") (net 1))
 (segment (start 113.399 98.851) (end 120 92.25) (width 0.2) (layer "B.Cu") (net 1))
 (segment (start 113.25 111.35) (end 113.35 111.25) (width 0.2) (layer "F.Cu") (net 31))
 (segment (start 91.75 107.5) (end 91.75 114.5) (width 0.2) (layer "F.Cu") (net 31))
 (segment (start 95.5 103.75) (end 91.75 107.5) (width 0.2) (layer "F.Cu") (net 31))
 (segment (start 117.91 83.23) (end 103.995326 83.23) (width 0.2) (layer "F.Cu") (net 31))
 (segment (start 113.25 114.75) (end 113.25 111.35) (width 0.2) (layer "F.Cu") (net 31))
 (segment (start 91.75 114.5) (end 93 115.75) (width 0.2) (layer "F.Cu") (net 31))
 (segment (start 101.5 85.725326) (end 101.5 102.25) (width 0.2) (layer "F.Cu") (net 31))
 (segment (start 103.995326 83.23) (end 101.5 85.725326) (width 0.2) (layer "F.Cu") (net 31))
 (segment (start 101.5 102.25) (end 100 103.75) (width 0.2) (layer "F.Cu") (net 31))
 (segment (start 100 103.75) (end 95.5 103.75) (width 0.2) (layer "F.Cu") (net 31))
 (segment (start 93 115.75) (end 112.25 115.75) (width 0.2) (layer "F.Cu") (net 31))
 (segment (start 112.25 115.75) (end 113.25 114.75) (width 0.2) (layer "F.Cu") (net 31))
 (segment (start 117.665 101.203) (end 122.938 95.93) (width 0.2) (layer "F.Cu") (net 17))
 (segment (start 103.55 110.148) (end 112.495 101.203) (width 0.2) (layer "F.Cu") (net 17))
 (segment (start 122.938 95.93) (end 135.41 95.93) (width 0.2) (layer "F.Cu") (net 17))
 (segment (start 112.495 101.203) (end 117.665 101.203) (width 0.2) (layer "F.Cu") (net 17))
 (segment (start 103.55 111.25) (end 103.55 110.148) (width 0.2) (layer "F.Cu") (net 17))
 (segment (start 132.8 97.2) (end 135.41 97.2) (width 0.2) (layer "F.Cu") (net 18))
 (segment (start 134.359 99.543) (end 134.359 97.301) (width 0.2) (layer "F.Cu") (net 18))
 (segment (start 135.41 88.31) (end 133.19 88.31) (width 0.2) (layer "F.Cu") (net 18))
 (segment (start 134.46 97.2) (end 135.41 97.2) (width 0.2) (layer "F.Cu") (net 18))
 (segment (start 104.25 111.25) (end 104.25 110.05) (width 0.2) (layer "F.Cu") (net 18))
 (segment (start 132.5 89) (end 132.5 89.75) (width 0.2) (layer "F.Cu") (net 18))
 (segment (start 104.25 110.05) (end 112.696 101.604) (width 0.2) (layer "F.Cu") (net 18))
 (segment (start 132.298 101.604) (end 134.359 99.543) (width 0.2) (layer "F.Cu") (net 18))
 (segment (start 133.19 88.31) (end 132.5 89) (width 0.2) (layer "F.Cu") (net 18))
 (segment (start 134.359 97.301) (end 134.46 97.2) (width 0.2) (layer "F.Cu") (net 18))
 (segment (start 112.696 101.604) (end 132.298 101.604) (width 0.2) (layer "F.Cu") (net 18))
 (segment (start 132.75 97.25) (end 132.8 97.2) (width 0.2) (layer "F.Cu") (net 18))
 (via (at 132.5 89.75) (size 0.6) (drill 0.3) (layers "F.Cu" "B.Cu") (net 18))
 (via (at 132.75 97.25) (size 0.6) (drill 0.3) (layers "F.Cu" "B.Cu") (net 18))
 (segment (start 132.5 89.75) (end 132.5 97) (width 0.2) (layer "B.Cu") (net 18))
 (segment (start 132.5 97) (end 132.75 97.25) (width 0.2) (layer "B.Cu") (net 18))
 (segment (start 130 84) (end 130.77 83.23) (width 0.2) (layer "F.Cu") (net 19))
 (segment (start 104.95 111.25) (end 104.95 110.148) (width 0.2) (layer "F.Cu") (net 19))
 (segment (start 130.77 83.23) (end 135.41 83.23) (width 0.2) (layer "F.Cu") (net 19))
 (segment (start 104.95 110.148) (end 110.848 104.25) (width 0.2) (layer "F.Cu") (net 19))
 (segment (start 110.848 104.25) (end 114 104.25) (width 0.2) (layer "F.Cu") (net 19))
 (via (at 114 104.25) (size 0.6) (drill 0.3) (layers "F.Cu" "B.Cu") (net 19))
 (via (at 130 84) (size 0.6) (drill 0.3) (layers "F.Cu" "B.Cu") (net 19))
 (segment (start 114.167443 104.25) (end 130 88.417443) (width 0.2) (layer "B.Cu") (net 19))
 (segment (start 114 104.25) (end 114.167443 104.25) (width 0.2) (layer "B.Cu") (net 19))
 (segment (start 130 88.417443) (end 130 84) (width 0.2) (layer "B.Cu") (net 19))
 (segment (start 124.792 93.39) (end 135.41 93.39) (width 0.2) (layer "F.Cu") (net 16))
 (segment (start 102.85 111.25) (end 102.85 100.802) (width 0.2) (layer "F.Cu") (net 16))
 (segment (start 102.85 100.802) (end 117.38 100.802) (width 0.2) (layer "F.Cu") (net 16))
 (segment (start 117.38 100.802) (end 124.792 93.39) (width 0.2) (layer "F.Cu") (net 16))
 (segment (start 123.98 113.3) (end 133.7 113.3) (width 0.2) (layer "F.Cu") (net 4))
 (segment (start 126.52 113.3) (end 126.125001 113.3) (width 0.2) (layer "F.Cu") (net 4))
 (segment (start 125.824 112.998999) (end 125.824 109.83113) (width 0.2) (layer "F.Cu") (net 4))
 (segment (start 123.98 109.3) (end 126.52 109.3) (width 0.2) (layer "F.Cu") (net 4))
 (segment (start 126.35513 109.3) (end 126.52 109.3) (width 0.2) (layer "F.Cu") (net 4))
 (segment (start 125.824 109.83113) (end 126.35513 109.3) (width 0.2) (layer "F.Cu") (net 4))
 (segment (start 126.125001 113.3) (end 125.824 112.998999) (width 0.2) (layer "F.Cu") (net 4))
 (segment (start 133.7 113.3) (end 133.95 113.55) (width 0.2) (layer "F.Cu") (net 4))
 (segment (start 164.95 113.55) (end 168.5 110) (width 0.2) (layer "F.Cu") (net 4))
 (segment (start 168.5 110) (end 168.5 108.75) (width 0.2) (layer "F.Cu") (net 4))
 (segment (start 133.95 113.55) (end 164.95 113.55) (width 0.2) (layer "F.Cu") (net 4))
 (segment (start 102.75 85) (end 103.25 84.5) (width 0.2) (layer "F.Cu") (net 2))
 (segment (start 144.9 110) (end 147.9 107) (width 0.2) (layer "F.Cu") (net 2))
 (segment (start 144.75 110) (end 144.9 110) (width 0.2) (layer "F.Cu") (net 2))
 (segment (start 150.749999 108.75) (end 149.5 108.75) (width 0.2) (layer "F.Cu") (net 2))
 (segment (start 149.150001 108.75) (end 149.5 108.75) (width 0.2) (layer "F.Cu") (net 2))
 (segment (start 152 107) (end 152 107.499999) (width 0.2) (layer "F.Cu") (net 2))
 (segment (start 147.9 107) (end 147.9 107.499999) (width 0.2) (layer "F.Cu") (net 2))
 (segment (start 152 107.499999) (end 150.749999 108.75) (width 0.2) (layer "F.Cu") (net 2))
 (segment (start 147.9 107.499999) (end 149.150001 108.75) (width 0.2) (layer "F.Cu") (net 2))
 (segment (start 103.25 84.5) (end 117.91 84.5) (width 0.2) (layer "F.Cu") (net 2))
 (segment (start 149.5 108.75) (end 165.96 108.75) (width 0.2) (layer "F.Cu") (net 2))
 (via (at 144.75 110) (size 0.6) (drill 0.3) (layers "F.Cu" "B.Cu") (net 2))
 (via (at 102.75 85) (size 0.2) (drill 0.2) (layers "F.Cu" "B.Cu") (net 2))
 (segment (start 144.75 110) (end 114.192484 110) (width 0.2) (layer "B.Cu") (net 2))
 (segment (start 102.75 98.557516) (end 102.75 85) (width 0.2) (layer "B.Cu") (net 2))
 (segment (start 114.192484 110) (end 102.75 98.557516) (width 0.2) (layer "B.Cu") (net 2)))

